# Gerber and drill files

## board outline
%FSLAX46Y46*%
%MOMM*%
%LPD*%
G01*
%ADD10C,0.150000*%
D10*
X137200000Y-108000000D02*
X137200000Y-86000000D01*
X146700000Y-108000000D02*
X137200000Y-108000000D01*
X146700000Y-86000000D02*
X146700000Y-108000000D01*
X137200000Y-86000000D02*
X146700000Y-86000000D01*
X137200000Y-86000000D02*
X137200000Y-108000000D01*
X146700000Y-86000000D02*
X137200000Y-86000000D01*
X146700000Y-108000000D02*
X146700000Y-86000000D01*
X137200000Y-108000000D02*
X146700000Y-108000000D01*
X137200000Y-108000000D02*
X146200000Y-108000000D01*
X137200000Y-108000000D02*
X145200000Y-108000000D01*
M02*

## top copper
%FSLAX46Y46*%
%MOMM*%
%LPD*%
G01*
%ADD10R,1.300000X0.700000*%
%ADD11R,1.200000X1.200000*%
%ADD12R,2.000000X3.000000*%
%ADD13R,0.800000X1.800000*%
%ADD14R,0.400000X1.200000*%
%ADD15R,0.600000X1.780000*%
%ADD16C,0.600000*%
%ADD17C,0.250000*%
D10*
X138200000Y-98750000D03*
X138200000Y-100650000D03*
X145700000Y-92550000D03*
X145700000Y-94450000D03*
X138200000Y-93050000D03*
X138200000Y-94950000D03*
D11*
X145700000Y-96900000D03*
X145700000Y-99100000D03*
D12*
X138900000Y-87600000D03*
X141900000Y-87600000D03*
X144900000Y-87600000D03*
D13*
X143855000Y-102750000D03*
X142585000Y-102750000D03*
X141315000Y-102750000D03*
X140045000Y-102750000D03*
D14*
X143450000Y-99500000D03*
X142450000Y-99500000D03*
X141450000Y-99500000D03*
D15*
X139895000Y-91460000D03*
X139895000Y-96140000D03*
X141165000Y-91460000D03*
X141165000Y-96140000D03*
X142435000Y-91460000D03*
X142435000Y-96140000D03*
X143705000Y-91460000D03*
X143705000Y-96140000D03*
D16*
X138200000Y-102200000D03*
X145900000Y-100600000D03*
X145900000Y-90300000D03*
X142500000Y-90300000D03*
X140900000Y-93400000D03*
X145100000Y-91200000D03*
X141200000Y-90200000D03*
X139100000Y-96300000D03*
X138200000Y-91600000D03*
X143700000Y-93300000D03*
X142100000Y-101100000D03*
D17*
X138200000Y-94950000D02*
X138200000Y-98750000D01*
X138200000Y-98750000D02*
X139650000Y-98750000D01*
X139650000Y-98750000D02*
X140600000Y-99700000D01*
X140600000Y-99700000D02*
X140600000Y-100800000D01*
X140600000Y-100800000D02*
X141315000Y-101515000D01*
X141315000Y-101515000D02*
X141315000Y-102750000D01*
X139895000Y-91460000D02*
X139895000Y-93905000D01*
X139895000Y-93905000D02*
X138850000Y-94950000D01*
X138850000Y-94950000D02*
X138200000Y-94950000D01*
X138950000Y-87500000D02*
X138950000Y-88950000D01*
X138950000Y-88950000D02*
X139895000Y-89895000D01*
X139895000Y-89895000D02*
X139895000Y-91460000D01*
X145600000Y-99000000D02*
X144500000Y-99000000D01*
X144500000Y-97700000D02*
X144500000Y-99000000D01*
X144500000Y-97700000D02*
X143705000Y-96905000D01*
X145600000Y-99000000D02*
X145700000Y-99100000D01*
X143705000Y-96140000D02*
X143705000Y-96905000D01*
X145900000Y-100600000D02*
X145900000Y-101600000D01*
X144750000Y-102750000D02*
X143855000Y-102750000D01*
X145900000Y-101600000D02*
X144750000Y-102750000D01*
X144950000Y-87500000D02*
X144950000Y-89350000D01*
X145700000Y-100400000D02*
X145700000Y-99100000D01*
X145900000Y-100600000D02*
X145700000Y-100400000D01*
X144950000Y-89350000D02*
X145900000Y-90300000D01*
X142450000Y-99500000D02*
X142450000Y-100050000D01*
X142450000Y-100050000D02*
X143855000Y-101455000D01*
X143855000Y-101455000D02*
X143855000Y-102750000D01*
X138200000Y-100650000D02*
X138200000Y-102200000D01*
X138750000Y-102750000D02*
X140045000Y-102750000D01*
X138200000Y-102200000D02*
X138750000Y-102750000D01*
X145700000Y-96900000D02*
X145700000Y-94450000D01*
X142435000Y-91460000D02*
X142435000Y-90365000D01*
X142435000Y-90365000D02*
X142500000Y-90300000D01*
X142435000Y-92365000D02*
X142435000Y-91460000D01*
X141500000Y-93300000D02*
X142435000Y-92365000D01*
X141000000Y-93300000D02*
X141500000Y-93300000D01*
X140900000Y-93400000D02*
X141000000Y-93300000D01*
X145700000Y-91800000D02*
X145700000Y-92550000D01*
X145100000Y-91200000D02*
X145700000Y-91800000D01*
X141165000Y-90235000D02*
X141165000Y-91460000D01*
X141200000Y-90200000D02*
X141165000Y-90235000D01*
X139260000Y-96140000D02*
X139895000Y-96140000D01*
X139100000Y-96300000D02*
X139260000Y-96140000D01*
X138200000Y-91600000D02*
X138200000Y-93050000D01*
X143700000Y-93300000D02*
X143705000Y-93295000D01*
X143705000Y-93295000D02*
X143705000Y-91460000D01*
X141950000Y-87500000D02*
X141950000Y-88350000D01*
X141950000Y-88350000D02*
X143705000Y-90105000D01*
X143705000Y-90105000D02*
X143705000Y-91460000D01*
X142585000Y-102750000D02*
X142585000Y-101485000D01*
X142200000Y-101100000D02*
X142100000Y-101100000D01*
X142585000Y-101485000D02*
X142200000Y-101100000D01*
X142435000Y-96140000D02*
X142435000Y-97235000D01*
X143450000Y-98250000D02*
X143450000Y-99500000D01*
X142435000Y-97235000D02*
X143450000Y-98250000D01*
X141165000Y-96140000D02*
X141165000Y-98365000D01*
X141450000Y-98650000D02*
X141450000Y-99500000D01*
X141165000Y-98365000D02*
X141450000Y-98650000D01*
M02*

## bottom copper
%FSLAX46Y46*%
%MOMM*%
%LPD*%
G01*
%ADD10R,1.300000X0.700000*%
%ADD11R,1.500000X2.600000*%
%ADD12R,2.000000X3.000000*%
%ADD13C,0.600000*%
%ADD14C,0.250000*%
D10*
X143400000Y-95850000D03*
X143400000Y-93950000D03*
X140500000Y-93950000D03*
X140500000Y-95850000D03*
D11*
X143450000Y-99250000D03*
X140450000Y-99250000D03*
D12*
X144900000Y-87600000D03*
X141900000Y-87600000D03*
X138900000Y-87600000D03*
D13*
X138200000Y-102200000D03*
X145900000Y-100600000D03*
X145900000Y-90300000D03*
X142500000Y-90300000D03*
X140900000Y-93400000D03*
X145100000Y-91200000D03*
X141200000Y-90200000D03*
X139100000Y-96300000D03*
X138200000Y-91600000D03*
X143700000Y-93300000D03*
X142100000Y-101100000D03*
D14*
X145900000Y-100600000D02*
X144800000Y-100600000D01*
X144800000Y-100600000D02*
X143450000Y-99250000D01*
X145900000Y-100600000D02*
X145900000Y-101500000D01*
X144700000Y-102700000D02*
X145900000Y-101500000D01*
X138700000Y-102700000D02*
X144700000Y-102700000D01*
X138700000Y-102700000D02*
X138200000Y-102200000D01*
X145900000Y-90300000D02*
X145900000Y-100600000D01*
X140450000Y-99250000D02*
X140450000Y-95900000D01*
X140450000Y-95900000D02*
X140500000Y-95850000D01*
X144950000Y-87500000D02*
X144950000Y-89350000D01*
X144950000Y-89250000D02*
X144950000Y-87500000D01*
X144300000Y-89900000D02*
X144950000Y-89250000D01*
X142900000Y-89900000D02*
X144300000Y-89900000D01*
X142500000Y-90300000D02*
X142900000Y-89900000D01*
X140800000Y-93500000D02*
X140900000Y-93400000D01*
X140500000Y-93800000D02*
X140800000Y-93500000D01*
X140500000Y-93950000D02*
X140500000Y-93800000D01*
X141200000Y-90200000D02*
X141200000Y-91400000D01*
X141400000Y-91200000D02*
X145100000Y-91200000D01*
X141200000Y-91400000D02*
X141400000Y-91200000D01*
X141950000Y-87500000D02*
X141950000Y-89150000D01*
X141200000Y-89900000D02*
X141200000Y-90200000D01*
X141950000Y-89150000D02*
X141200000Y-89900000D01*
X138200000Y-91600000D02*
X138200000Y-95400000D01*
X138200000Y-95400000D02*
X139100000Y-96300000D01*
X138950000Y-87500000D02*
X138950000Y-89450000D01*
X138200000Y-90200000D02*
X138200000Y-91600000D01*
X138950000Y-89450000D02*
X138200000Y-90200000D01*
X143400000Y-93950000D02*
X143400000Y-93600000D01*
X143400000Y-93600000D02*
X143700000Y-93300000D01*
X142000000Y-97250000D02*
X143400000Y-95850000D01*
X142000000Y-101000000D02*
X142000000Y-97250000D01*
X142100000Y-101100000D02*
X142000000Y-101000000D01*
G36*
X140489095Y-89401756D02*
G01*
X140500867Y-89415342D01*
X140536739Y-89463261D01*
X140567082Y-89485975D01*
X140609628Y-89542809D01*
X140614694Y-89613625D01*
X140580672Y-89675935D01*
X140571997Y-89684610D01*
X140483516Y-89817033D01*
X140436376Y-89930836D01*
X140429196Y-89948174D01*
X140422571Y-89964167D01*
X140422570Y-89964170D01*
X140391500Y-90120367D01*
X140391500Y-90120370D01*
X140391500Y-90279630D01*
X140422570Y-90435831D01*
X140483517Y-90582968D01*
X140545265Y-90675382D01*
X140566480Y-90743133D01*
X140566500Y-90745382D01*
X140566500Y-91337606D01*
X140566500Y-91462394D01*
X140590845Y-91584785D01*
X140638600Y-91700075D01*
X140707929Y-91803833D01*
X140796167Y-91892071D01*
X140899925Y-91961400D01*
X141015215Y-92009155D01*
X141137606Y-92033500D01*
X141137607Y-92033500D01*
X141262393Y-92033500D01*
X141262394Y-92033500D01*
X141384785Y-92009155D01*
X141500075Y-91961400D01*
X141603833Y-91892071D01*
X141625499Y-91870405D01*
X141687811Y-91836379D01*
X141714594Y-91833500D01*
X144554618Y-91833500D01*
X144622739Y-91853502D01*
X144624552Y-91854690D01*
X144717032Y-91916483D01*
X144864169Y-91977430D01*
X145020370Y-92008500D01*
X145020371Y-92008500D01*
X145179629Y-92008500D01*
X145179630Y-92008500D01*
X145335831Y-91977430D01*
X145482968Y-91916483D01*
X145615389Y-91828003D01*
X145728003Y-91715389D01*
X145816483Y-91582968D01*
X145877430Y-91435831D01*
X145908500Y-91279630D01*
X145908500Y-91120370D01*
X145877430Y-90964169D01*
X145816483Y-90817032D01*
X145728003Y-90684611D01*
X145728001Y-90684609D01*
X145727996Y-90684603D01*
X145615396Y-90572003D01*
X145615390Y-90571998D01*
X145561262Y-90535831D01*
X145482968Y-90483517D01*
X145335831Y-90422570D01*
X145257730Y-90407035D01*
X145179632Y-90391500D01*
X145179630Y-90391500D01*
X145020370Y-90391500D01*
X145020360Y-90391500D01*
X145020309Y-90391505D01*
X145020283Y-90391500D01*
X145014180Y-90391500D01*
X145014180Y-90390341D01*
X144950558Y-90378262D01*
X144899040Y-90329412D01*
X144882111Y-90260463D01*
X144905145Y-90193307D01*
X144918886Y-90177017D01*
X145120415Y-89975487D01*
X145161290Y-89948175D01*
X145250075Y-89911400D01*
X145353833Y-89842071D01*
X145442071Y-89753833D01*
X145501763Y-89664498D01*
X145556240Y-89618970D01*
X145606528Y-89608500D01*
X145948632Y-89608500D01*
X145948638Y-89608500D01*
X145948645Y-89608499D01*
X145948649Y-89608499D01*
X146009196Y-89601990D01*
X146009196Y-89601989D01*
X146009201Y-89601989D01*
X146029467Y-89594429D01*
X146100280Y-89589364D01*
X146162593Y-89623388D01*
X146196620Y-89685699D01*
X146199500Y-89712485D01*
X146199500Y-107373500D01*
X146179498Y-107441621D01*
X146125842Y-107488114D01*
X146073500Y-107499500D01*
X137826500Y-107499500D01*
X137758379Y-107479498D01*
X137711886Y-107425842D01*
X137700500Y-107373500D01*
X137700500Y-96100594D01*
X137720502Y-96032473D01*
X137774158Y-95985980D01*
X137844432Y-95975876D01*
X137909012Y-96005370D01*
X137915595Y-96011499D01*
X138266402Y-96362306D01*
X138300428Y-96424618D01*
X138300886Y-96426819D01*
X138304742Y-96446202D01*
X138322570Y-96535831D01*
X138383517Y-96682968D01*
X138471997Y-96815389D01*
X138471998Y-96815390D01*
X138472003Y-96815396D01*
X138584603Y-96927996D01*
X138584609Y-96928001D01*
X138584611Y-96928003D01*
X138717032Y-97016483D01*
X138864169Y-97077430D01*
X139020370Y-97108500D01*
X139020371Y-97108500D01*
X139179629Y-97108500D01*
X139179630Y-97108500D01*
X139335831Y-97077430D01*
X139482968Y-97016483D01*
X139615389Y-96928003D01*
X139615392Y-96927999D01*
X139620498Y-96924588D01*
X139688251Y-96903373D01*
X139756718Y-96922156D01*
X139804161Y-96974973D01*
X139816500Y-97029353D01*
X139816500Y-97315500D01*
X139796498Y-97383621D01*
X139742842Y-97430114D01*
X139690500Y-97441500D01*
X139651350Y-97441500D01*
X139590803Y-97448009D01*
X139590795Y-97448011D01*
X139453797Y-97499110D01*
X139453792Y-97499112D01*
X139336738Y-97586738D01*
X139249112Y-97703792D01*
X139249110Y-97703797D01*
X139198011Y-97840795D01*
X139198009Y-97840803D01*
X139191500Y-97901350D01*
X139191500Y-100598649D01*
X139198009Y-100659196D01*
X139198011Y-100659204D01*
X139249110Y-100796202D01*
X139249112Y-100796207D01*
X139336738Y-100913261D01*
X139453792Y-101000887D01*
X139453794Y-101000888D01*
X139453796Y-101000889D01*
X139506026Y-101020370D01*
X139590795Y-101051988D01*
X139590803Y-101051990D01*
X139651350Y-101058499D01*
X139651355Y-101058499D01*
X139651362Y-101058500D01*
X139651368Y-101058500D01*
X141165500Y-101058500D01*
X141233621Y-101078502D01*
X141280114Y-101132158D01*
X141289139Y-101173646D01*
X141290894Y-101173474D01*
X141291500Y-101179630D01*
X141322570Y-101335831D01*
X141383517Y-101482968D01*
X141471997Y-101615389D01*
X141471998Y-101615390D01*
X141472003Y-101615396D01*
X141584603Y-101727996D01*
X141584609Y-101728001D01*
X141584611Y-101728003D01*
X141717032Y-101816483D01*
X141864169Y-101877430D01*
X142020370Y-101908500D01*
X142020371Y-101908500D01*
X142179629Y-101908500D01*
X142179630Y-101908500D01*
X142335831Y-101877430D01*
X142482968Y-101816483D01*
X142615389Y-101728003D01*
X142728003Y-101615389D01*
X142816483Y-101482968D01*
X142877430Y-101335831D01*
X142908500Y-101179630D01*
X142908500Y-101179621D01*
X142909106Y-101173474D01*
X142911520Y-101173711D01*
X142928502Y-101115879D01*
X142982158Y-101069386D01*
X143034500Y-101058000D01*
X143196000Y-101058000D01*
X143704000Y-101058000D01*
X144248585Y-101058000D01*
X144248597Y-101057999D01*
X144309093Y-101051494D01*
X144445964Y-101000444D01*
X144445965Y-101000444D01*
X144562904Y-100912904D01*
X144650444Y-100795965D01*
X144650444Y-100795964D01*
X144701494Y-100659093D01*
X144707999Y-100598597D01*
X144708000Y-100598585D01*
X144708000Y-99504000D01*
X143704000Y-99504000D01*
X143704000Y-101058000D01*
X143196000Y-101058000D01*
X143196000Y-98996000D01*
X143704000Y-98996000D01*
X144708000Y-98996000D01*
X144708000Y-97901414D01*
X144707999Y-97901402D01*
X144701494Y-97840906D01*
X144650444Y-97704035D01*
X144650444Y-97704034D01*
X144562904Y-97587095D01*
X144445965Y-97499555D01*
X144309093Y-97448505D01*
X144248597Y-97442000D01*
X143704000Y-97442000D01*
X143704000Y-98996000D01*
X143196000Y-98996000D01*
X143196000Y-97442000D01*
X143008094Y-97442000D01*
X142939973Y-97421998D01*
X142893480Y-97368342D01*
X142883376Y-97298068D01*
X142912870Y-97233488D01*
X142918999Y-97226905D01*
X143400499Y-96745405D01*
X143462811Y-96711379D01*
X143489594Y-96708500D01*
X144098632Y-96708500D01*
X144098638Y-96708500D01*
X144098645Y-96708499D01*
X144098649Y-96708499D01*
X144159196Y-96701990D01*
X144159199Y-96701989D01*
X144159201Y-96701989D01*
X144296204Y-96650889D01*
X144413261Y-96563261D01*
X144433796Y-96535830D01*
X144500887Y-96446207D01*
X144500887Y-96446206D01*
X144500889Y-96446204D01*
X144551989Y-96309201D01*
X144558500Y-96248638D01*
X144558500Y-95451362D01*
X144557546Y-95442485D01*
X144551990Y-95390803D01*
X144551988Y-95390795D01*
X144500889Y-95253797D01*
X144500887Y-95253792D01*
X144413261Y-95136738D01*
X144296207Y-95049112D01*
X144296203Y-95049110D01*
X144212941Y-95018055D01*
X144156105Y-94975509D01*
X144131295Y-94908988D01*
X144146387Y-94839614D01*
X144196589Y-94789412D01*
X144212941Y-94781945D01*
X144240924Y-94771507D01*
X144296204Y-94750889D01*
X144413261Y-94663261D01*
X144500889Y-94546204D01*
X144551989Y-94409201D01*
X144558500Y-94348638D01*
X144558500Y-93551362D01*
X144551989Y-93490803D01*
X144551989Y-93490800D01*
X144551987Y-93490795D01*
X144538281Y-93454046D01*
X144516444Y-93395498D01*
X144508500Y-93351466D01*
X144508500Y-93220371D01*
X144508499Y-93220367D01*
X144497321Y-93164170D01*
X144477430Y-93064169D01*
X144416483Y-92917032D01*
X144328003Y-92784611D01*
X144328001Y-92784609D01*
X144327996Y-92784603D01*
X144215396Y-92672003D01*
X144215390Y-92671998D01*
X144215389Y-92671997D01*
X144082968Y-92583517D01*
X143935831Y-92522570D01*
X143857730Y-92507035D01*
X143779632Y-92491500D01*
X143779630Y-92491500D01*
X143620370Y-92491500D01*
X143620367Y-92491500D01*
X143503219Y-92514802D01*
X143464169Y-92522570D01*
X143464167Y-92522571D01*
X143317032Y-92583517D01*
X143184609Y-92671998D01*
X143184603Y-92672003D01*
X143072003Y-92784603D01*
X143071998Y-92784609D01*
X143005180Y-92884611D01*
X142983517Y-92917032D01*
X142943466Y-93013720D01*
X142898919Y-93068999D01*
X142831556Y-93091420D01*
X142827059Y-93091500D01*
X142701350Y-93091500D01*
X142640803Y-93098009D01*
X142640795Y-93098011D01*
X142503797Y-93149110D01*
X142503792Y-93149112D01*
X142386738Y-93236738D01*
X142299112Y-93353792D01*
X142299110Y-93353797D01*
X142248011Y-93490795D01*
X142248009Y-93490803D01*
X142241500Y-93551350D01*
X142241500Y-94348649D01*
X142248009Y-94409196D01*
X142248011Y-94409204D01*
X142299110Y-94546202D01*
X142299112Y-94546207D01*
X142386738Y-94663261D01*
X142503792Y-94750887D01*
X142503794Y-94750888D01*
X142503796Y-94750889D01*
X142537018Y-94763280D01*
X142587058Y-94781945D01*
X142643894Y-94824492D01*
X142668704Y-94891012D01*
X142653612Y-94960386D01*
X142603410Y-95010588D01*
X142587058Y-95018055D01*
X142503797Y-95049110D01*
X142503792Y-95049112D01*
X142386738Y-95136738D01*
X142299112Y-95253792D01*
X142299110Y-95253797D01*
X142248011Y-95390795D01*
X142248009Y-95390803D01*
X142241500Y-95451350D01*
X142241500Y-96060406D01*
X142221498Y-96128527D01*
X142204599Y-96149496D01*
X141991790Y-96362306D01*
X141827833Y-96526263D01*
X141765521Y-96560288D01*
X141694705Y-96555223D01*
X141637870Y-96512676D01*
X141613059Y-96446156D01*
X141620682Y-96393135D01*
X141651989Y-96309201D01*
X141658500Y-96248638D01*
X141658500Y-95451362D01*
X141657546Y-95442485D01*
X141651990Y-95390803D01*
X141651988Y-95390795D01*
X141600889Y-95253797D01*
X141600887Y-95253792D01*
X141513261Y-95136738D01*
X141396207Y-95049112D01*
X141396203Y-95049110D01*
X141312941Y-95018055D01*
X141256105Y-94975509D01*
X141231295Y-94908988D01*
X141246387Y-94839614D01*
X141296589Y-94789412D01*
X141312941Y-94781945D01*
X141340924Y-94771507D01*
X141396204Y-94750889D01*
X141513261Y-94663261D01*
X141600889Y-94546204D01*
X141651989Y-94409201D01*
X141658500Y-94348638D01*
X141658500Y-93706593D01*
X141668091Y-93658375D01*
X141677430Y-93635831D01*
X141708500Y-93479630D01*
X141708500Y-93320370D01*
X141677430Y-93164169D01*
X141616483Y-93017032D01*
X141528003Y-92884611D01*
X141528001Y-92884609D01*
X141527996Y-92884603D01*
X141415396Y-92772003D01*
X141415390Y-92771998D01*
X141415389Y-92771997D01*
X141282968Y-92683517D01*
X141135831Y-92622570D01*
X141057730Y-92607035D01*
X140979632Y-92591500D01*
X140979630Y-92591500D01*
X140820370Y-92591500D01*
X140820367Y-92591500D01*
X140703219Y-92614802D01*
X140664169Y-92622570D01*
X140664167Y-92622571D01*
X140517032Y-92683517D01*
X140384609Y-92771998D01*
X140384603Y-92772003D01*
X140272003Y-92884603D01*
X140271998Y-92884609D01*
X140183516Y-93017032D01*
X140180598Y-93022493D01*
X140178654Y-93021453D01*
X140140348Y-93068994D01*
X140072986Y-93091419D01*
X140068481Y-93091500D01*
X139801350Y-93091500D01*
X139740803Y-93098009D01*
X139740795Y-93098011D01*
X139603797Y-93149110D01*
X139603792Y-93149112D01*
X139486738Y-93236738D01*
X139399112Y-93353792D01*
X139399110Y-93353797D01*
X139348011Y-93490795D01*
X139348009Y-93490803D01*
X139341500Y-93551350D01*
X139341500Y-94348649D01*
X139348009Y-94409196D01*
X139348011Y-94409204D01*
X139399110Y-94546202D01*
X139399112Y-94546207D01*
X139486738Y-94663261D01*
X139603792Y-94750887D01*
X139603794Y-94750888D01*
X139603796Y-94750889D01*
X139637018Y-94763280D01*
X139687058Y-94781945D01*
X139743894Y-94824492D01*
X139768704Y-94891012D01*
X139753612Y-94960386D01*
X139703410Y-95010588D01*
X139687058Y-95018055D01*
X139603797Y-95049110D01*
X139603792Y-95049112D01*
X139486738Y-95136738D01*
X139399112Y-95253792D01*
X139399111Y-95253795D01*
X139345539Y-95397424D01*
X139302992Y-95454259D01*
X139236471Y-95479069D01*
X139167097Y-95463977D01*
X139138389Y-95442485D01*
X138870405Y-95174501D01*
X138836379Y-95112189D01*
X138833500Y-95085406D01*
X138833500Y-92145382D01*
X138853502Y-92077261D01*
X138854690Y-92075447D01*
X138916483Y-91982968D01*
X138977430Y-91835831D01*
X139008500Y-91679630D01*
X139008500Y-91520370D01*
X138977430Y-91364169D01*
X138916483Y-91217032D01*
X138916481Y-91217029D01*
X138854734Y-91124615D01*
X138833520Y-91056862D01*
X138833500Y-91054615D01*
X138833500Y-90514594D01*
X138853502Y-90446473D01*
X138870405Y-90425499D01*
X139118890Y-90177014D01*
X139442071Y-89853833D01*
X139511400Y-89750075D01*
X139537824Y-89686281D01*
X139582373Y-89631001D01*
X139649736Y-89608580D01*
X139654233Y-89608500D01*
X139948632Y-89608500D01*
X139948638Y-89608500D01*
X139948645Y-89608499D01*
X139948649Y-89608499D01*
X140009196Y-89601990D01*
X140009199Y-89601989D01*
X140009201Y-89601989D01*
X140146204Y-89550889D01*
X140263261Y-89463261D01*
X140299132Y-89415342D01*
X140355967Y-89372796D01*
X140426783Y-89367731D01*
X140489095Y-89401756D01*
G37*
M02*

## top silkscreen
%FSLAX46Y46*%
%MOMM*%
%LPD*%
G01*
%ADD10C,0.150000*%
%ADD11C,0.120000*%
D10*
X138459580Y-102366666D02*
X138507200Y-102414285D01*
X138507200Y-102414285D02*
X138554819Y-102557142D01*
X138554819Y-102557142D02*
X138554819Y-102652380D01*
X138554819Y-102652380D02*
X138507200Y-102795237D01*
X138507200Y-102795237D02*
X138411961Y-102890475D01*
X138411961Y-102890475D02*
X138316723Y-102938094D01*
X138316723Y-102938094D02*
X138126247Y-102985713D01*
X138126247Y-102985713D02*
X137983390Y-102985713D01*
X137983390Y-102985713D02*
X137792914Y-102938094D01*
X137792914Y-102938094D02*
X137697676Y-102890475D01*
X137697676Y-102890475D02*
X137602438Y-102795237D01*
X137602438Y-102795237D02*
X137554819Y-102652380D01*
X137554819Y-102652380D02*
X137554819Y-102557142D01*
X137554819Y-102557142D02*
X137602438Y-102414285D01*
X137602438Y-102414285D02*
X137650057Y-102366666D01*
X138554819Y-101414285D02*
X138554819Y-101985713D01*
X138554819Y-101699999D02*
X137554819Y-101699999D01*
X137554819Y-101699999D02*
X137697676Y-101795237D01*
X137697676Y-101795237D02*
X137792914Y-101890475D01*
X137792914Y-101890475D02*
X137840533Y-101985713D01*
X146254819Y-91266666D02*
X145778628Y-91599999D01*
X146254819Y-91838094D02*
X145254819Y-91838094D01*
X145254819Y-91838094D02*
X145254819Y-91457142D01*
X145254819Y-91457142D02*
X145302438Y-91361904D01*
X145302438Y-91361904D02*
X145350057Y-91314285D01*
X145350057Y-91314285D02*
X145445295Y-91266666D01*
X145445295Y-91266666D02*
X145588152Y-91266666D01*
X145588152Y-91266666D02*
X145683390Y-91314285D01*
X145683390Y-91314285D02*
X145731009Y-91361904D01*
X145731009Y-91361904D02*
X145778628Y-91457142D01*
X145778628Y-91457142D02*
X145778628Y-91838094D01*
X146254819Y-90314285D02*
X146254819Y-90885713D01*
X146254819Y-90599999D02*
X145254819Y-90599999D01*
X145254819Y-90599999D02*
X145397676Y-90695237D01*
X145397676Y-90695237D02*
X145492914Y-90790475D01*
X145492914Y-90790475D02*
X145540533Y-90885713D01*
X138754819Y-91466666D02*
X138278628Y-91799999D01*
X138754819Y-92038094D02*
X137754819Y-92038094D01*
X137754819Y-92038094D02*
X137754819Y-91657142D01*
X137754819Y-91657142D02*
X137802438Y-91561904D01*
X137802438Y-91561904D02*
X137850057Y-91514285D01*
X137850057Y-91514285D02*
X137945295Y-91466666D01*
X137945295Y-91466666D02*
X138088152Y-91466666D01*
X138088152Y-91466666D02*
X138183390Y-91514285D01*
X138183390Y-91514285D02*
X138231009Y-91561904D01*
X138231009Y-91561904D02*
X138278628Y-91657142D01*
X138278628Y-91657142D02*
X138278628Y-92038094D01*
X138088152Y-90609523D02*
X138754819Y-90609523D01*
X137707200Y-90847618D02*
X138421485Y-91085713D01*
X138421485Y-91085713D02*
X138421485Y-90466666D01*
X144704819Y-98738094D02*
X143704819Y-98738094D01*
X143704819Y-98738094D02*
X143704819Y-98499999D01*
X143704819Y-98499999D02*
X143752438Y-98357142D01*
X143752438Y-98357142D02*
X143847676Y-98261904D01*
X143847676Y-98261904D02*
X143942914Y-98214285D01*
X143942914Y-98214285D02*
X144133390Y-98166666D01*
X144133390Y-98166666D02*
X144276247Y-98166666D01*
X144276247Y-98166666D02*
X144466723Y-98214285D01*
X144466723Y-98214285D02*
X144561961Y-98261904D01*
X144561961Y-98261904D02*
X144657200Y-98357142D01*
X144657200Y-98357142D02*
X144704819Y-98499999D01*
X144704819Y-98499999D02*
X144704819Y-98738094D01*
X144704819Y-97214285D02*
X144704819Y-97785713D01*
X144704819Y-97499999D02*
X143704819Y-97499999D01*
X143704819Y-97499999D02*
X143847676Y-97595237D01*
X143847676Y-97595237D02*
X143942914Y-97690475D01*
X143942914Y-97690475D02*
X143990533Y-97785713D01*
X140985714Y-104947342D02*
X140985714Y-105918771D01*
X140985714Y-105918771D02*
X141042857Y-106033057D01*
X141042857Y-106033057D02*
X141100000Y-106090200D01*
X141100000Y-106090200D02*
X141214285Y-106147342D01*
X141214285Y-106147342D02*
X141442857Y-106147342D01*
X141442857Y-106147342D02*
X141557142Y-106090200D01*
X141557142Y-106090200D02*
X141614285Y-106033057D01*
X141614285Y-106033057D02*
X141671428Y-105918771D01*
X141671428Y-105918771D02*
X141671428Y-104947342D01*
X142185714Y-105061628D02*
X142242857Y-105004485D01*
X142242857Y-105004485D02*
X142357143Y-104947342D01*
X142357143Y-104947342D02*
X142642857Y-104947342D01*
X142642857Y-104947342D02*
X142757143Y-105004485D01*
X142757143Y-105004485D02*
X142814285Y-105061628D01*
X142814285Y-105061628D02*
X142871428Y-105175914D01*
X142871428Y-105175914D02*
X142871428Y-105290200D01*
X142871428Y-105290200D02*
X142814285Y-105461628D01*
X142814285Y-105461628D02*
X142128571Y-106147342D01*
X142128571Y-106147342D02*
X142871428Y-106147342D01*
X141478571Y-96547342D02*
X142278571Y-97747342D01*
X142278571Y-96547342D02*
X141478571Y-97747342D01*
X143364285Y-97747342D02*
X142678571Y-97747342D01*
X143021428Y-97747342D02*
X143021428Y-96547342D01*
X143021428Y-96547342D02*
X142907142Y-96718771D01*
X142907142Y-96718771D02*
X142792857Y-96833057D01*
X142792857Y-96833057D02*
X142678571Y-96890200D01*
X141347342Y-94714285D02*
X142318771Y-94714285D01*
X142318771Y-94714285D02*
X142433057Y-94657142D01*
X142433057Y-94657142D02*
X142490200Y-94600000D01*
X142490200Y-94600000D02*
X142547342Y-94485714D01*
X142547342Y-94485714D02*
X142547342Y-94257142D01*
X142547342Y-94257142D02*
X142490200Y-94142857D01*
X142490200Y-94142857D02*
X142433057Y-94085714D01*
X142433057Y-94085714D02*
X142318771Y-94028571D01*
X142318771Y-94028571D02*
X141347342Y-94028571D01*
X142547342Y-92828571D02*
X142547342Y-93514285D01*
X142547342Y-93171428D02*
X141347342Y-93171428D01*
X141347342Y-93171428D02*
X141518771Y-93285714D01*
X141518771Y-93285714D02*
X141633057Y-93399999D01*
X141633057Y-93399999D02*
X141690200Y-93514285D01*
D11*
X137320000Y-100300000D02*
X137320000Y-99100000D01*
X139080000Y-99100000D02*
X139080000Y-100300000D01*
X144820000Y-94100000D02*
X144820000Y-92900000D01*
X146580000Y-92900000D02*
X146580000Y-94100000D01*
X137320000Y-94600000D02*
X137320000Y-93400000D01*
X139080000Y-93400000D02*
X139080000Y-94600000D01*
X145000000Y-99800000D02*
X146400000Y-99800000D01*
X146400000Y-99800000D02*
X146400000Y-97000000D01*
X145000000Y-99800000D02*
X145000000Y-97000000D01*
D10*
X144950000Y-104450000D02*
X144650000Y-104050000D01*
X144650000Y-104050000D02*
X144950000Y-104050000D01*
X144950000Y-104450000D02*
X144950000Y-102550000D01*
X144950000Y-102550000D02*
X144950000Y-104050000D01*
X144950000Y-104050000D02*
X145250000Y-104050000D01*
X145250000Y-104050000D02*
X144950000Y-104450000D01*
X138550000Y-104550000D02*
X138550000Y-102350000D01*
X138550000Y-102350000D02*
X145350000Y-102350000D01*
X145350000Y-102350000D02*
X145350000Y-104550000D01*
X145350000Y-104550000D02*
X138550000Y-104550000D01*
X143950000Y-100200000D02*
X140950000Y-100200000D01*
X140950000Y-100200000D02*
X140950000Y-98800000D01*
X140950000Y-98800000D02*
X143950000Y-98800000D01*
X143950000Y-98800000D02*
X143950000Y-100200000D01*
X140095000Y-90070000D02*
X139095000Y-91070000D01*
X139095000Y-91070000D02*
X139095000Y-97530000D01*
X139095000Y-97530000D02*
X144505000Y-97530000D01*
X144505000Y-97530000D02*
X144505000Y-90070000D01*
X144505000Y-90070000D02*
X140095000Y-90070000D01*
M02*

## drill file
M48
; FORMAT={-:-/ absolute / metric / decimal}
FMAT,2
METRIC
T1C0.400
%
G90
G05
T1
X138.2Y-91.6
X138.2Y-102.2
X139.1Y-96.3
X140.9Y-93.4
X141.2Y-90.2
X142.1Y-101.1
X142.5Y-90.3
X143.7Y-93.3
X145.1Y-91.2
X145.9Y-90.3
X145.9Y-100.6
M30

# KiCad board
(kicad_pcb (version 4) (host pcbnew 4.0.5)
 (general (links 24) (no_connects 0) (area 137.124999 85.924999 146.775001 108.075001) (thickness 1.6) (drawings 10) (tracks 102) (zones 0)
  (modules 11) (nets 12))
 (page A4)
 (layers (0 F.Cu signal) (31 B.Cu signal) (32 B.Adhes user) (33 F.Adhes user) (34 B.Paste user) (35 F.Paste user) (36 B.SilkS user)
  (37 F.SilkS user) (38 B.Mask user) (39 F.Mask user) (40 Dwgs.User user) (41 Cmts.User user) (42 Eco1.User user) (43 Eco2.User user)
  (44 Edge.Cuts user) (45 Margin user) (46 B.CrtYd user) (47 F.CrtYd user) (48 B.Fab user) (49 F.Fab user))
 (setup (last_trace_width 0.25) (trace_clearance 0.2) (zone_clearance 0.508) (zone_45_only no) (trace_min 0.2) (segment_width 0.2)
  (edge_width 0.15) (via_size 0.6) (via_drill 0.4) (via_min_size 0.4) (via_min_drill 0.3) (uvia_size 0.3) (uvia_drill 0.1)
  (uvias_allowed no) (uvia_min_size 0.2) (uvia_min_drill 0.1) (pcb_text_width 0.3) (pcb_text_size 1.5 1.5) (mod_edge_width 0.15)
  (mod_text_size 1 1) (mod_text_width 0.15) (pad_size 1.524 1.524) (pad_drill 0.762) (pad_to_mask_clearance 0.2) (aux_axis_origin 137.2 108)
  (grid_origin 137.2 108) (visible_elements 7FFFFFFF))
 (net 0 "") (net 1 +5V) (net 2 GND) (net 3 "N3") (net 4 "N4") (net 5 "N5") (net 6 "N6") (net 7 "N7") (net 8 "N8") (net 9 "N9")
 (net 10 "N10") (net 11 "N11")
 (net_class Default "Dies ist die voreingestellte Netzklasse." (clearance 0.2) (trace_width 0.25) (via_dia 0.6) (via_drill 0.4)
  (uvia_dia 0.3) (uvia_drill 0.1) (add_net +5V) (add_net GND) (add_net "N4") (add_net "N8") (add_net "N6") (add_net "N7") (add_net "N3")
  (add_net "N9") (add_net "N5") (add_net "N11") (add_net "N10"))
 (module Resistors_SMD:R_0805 (layer F.Cu) (at 138.2 99.7 270)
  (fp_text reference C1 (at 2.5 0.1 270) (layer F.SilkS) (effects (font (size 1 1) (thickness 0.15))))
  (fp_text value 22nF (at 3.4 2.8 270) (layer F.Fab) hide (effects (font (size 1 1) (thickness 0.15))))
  (fp_line (start 0.6 0.88) (end -0.6 0.88) (layer F.SilkS) (width 0.12))
  (fp_line (start -0.6 -0.88) (end 0.6 -0.88) (layer F.SilkS) (width 0.12))
  (pad 1 smd rect (at -0.95 0 270) (size 0.7 1.3) (layers F.Cu F.Paste F.Mask) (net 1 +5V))
  (pad 2 smd rect (at 0.95 0 270) (size 0.7 1.3) (layers F.Cu F.Paste F.Mask) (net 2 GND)))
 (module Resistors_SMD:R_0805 (layer F.Cu) (at 145.7 93.5 270)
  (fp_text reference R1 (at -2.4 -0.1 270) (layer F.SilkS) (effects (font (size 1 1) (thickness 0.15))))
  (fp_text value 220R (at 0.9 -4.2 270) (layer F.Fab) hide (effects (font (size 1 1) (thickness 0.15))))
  (fp_line (start 0.6 0.88) (end -0.6 0.88) (layer F.SilkS) (width 0.12))
  (fp_line (start -0.6 -0.88) (end 0.6 -0.88) (layer F.SilkS) (width 0.12))
  (pad 1 smd rect (at -0.95 0 270) (size 0.7 1.3) (layers F.Cu F.Paste F.Mask) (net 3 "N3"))
  (pad 2 smd rect (at 0.95 0 270) (size 0.7 1.3) (layers F.Cu F.Paste F.Mask) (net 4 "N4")))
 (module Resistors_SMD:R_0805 (layer B.Cu) (at 143.4 94.9 90)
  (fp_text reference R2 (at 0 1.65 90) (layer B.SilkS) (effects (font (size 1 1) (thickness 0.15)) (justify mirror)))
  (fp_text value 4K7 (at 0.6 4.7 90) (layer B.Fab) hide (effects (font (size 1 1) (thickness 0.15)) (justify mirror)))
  (pad 1 smd rect (at -0.95 0 90) (size 0.7 1.3) (layers B.Cu B.Paste B.Mask) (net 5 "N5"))
  (pad 2 smd rect (at 0.95 0 90) (size 0.7 1.3) (layers B.Cu B.Paste B.Mask) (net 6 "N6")))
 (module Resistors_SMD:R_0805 (layer B.Cu) (at 140.5 94.9 270)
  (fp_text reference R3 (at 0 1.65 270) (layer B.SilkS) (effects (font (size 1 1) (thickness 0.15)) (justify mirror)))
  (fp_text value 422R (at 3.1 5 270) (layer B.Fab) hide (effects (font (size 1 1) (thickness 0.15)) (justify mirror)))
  (pad 1 smd rect (at -0.95 0 270) (size 0.7 1.3) (layers B.Cu B.Paste B.Mask) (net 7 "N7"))
  (pad 2 smd rect (at 0.95 0 270) (size 0.7 1.3) (layers B.Cu B.Paste B.Mask) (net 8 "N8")))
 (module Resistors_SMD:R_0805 (layer F.Cu) (at 138.2 94 270)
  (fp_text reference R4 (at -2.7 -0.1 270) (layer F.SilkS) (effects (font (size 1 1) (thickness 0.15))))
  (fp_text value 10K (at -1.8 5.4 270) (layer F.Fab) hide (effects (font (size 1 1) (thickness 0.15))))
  (fp_line (start 0.6 0.88) (end -0.6 0.88) (layer F.SilkS) (width 0.12))
  (fp_line (start -0.6 -0.88) (end 0.6 -0.88) (layer F.SilkS) (width 0.12))
  (pad 1 smd rect (at -0.95 0 270) (size 0.7 1.3) (layers F.Cu F.Paste F.Mask) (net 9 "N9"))
  (pad 2 smd rect (at 0.95 0 270) (size 0.7 1.3) (layers F.Cu F.Paste F.Mask) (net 1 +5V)))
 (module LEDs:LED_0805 (layer F.Cu) (at 145.7 98 90)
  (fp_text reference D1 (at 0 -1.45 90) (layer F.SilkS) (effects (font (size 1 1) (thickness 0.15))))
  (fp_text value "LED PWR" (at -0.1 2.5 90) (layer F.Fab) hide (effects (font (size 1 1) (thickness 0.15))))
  (fp_line (start -1.8 -0.7) (end -1.8 0.7) (layer F.SilkS) (width 0.12))
  (fp_line (start -1.8 0.7) (end 1 0.7) (layer F.SilkS) (width 0.12))
  (fp_line (start -1.8 -0.7) (end 1 -0.7) (layer F.SilkS) (width 0.12))
  (pad 2 smd rect (at 1.1 0 270) (size 1.2 1.2) (layers F.Cu F.Paste F.Mask) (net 4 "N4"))
  (pad 1 smd rect (at -1.1 0 270) (size 1.2 1.2) (layers F.Cu F.Paste F.Mask) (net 2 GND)))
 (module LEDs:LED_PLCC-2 (layer B.Cu) (at 141.95 99.25 180)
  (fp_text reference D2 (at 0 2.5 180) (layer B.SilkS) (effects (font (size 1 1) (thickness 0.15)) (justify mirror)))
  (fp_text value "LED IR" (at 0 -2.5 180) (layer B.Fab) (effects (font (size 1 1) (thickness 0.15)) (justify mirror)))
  (pad 1 smd rect (at -1.5 0 180) (size 1.5 2.6) (layers B.Cu B.Paste B.Mask) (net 2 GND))
  (pad 2 smd rect (at 1.5 0 180) (size 1.5 2.6) (layers B.Cu B.Paste B.Mask) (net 8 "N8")))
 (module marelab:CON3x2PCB (layer F.Cu) (at 141.9 87.6)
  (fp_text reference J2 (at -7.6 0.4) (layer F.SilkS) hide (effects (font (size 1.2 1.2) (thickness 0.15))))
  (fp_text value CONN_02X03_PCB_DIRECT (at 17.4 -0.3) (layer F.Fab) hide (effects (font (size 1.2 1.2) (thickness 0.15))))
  (pad 4 smd rect (at 3 0) (size 2 3) (layers *.Mask B.Cu B.Paste) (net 7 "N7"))
  (pad 5 smd rect (at 0 0) (size 2 3) (layers B.Cu F.Paste B.Mask) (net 3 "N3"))
  (pad 6 smd rect (at -3 0) (size 2 3) (layers B.Cu B.Paste B.Mask) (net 9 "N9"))
  (pad 1 smd rect (at -3 0) (size 2 3) (layers F.Cu F.Paste F.Mask) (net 1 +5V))
  (pad 2 smd rect (at 0 0) (size 2 3) (layers F.Cu F.Paste F.Mask) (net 6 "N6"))
  (pad 3 smd rect (at 3 0) (size 2 3) (layers F.Cu F.Paste F.Mask) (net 2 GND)))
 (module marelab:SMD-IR (layer F.Cu) (at 141.95 102.75 180)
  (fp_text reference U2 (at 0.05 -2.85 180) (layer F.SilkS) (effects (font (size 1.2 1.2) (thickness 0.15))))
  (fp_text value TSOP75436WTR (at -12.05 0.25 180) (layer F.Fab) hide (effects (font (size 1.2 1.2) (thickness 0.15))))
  (fp_line (start -3 -1.7) (end -2.7 -1.3) (layer F.SilkS) (width 0.15))
  (fp_line (start -2.7 -1.3) (end -3 -1.3) (layer F.SilkS) (width 0.15))
  (fp_line (start -3 -1.7) (end -3 0.2) (layer F.SilkS) (width 0.15))
  (fp_line (start -3 0.2) (end -3 -1.3) (layer F.SilkS) (width 0.15))
  (fp_line (start -3 -1.3) (end -3.3 -1.3) (layer F.SilkS) (width 0.15))
  (fp_line (start -3.3 -1.3) (end -3 -1.7) (layer F.SilkS) (width 0.15))
  (fp_line (start 3.4 -1.8) (end 3.4 0.4) (layer F.SilkS) (width 0.15))
  (fp_line (start 3.4 0.4) (end -3.4 0.4) (layer F.SilkS) (width 0.15))
  (fp_line (start -3.4 0.4) (end -3.4 -1.8) (layer F.SilkS) (width 0.15))
  (fp_line (start -3.4 -1.8) (end 3.4 -1.8) (layer F.SilkS) (width 0.15))
  (pad 4 smd rect (at -1.905 0 180) (size 0.8 1.8) (layers F.Cu F.Paste F.Mask) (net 2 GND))
  (pad 3 smd rect (at -0.635 0 180) (size 0.8 1.8) (layers F.Cu F.Paste F.Mask) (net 5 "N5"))
  (pad 2 smd rect (at 0.635 0 180) (size 0.8 1.8) (layers F.Cu F.Paste F.Mask) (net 1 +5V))
  (pad 1 smd rect (at 1.905 0 180) (size 0.8 1.8) (layers F.Cu F.Paste F.Mask) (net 2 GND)))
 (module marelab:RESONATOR (layer F.Cu) (at 142.45 99.5 180)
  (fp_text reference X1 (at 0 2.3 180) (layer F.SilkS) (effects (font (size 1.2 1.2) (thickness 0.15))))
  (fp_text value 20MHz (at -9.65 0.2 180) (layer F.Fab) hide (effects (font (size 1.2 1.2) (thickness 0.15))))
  (fp_line (start -1.5 -0.7) (end 1.5 -0.7) (layer F.SilkS) (width 0.15))
  (fp_line (start 1.5 -0.7) (end 1.5 0.7) (layer F.SilkS) (width 0.15))
  (fp_line (start 1.5 0.7) (end -1.5 0.7) (layer F.SilkS) (width 0.15))
  (fp_line (start -1.5 0.7) (end -1.5 -0.7) (layer F.SilkS) (width 0.15))
  (pad 1 smd rect (at -1 0 180) (size 0.4 1.2) (layers F.Cu F.Paste F.Mask) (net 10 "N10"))
  (pad 2 smd rect (at 0 0 180) (size 0.4 1.2) (layers F.Cu F.Paste F.Mask) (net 2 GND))
  (pad 3 smd rect (at 1 0 180) (size 0.4 1.2) (layers F.Cu F.Paste F.Mask) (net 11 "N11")))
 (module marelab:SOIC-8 (layer F.Cu) (at 141.8 93.8)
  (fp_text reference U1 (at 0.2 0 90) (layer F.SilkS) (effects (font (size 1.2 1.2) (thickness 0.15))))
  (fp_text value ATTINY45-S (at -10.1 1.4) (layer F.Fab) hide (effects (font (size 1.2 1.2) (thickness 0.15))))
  (fp_line (start -1.705 -3.73) (end -2.705 -2.73) (layer F.SilkS) (width 0.15))
  (fp_line (start -2.705 -2.73) (end -2.705 3.73) (layer F.SilkS) (width 0.15))
  (fp_line (start -2.705 3.73) (end 2.705 3.73) (layer F.SilkS) (width 0.15))
  (fp_line (start 2.705 3.73) (end 2.705 -3.73) (layer F.SilkS) (width 0.15))
  (fp_line (start 2.705 -3.73) (end -1.705 -3.73) (layer F.SilkS) (width 0.15))
  (pad 8 smd rect (at -1.905 -2.34) (size 0.6 1.78) (layers F.Cu F.Paste F.Mask) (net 1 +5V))
  (pad 1 smd rect (at -1.905 2.34) (size 0.6 1.78) (layers F.Cu F.Paste F.Mask) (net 9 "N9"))
  (pad 7 smd rect (at -0.635 -2.34) (size 0.6 1.78) (layers F.Cu F.Paste F.Mask) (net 3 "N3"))
  (pad 2 smd rect (at -0.635 2.34) (size 0.6 1.78) (layers F.Cu F.Paste F.Mask) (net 11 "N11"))
  (pad 6 smd rect (at 0.635 -2.34) (size 0.6 1.78) (layers F.Cu F.Paste F.Mask) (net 7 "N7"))
  (pad 3 smd rect (at 0.635 2.34) (size 0.6 1.78) (layers F.Cu F.Paste F.Mask) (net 10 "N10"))
  (pad 5 smd rect (at 1.905 -2.34) (size 0.6 1.78) (layers F.Cu F.Paste F.Mask) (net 6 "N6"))
  (pad 4 smd rect (at 1.905 2.34) (size 0.6 1.78) (layers F.Cu F.Paste F.Mask) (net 2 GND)))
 (gr_line (start 137.2 108) (end 137.2 86) (angle 90) (layer Edge.Cuts) (width 0.15))
 (gr_line (start 146.7 108) (end 137.2 108) (angle 90) (layer Edge.Cuts) (width 0.15))
 (gr_line (start 146.7 86) (end 146.7 108) (angle 90) (layer Edge.Cuts) (width 0.15))
 (gr_line (start 137.2 86) (end 146.7 86) (angle 90) (layer Edge.Cuts) (width 0.15))
 (gr_line (start 137.2 86) (end 137.2 108) (angle 90) (layer Edge.Cuts) (width 0.15))
 (gr_line (start 146.7 86) (end 137.2 86) (angle 90) (layer Edge.Cuts) (width 0.15))
 (gr_line (start 146.7 108) (end 146.7 86) (angle 90) (layer Edge.Cuts) (width 0.15))
 (gr_line (start 137.2 108) (end 146.7 108) (angle 90) (layer Edge.Cuts) (width 0.15))
 (gr_line (start 137.2 108) (end 146.2 108) (angle 90) (layer Edge.Cuts) (width 0.15))
 (gr_line (start 137.2 108) (end 145.2 108) (angle 90) (layer Edge.Cuts) (width 0.15))
 (segment (start 138.2 94.95) (end 138.2 98.75) (width 0.25) (layer F.Cu) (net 1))
 (segment (start 138.2 98.75) (end 139.65 98.75) (width 0.25) (layer F.Cu) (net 1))
 (segment (start 139.65 98.75) (end 140.6 99.7) (width 0.25) (layer F.Cu) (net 1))
 (segment (start 140.6 99.7) (end 140.6 100.8) (width 0.25) (layer F.Cu) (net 1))
 (segment (start 140.6 100.8) (end 141.315 101.515) (width 0.25) (layer F.Cu) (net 1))
 (segment (start 141.315 101.515) (end 141.315 102.75) (width 0.25) (layer F.Cu) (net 1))
 (segment (start 139.895 91.46) (end 139.895 93.905) (width 0.25) (layer F.Cu) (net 1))
 (segment (start 139.895 93.905) (end 138.85 94.95) (width 0.25) (layer F.Cu) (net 1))
 (segment (start 138.85 94.95) (end 138.2 94.95) (width 0.25) (layer F.Cu) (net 1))
 (segment (start 138.95 87.5) (end 138.95 88.95) (width 0.25) (layer F.Cu) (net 1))
 (segment (start 138.95 88.95) (end 139.895 89.895) (width 0.25) (layer F.Cu) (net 1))
 (segment (start 139.895 89.895) (end 139.895 91.46) (width 0.25) (layer F.Cu) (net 1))
 (segment (start 145.6 99) (end 144.5 99) (width 0.25) (layer F.Cu) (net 2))
 (segment (start 144.5 97.7) (end 144.5 99) (width 0.25) (layer F.Cu) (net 2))
 (segment (start 144.5 97.7) (end 143.705 96.905) (width 0.25) (layer F.Cu) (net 2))
 (segment (start 145.6 99) (end 145.7 99.1) (width 0.25) (layer F.Cu) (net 2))
 (segment (start 143.705 96.14) (end 143.705 96.905) (width 0.25) (layer F.Cu) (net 2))
 (segment (start 145.9 100.6) (end 144.8 100.6) (width 0.25) (layer B.Cu) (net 2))
 (segment (start 144.8 100.6) (end 143.45 99.25) (width 0.25) (layer B.Cu) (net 2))
 (via (at 138.2 102.2) (size 0.6) (drill 0.4) (layers F.Cu B.Cu) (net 2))
 (segment (start 145.9 100.6) (end 145.9 101.5) (width 0.25) (layer B.Cu) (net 2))
 (segment (start 144.7 102.7) (end 145.9 101.5) (width 0.25) (layer B.Cu) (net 2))
 (segment (start 138.7 102.7) (end 144.7 102.7) (width 0.25) (layer B.Cu) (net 2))
 (segment (start 138.7 102.7) (end 138.2 102.2) (width 0.25) (layer B.Cu) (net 2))
 (segment (start 145.9 100.6) (end 145.9 101.6) (width 0.25) (layer F.Cu) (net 2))
 (segment (start 144.75 102.75) (end 143.855 102.75) (width 0.25) (layer F.Cu) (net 2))
 (segment (start 145.9 101.6) (end 144.75 102.75) (width 0.25) (layer F.Cu) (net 2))
 (segment (start 144.95 87.5) (end 144.95 89.35) (width 0.25) (layer F.Cu) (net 2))
 (segment (start 145.7 100.4) (end 145.7 99.1) (width 0.25) (layer F.Cu) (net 2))
 (segment (start 145.9 100.6) (end 145.7 100.4) (width 0.25) (layer F.Cu) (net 2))
 (via (at 145.9 100.6) (size 0.6) (drill 0.4) (layers F.Cu B.Cu) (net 2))
 (segment (start 145.9 90.3) (end 145.9 100.6) (width 0.25) (layer B.Cu) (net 2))
 (via (at 145.9 90.3) (size 0.6) (drill 0.4) (layers F.Cu B.Cu) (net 2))
 (segment (start 144.95 89.35) (end 145.9 90.3) (width 0.25) (layer F.Cu) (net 2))
 (segment (start 142.45 99.5) (end 142.45 100.05) (width 0.25) (layer F.Cu) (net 2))
 (segment (start 142.45 100.05) (end 143.855 101.455) (width 0.25) (layer F.Cu) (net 2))
 (segment (start 143.855 101.455) (end 143.855 102.75) (width 0.25) (layer F.Cu) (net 2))
 (segment (start 138.2 100.65) (end 138.2 102.2) (width 0.25) (layer F.Cu) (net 2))
 (segment (start 138.75 102.75) (end 140.045 102.75) (width 0.25) (layer F.Cu) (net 2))
 (segment (start 138.2 102.2) (end 138.75 102.75) (width 0.25) (layer F.Cu) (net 2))
 (segment (start 145.7 96.9) (end 145.7 94.45) (width 0.25) (layer F.Cu) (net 4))
 (segment (start 140.45 99.25) (end 140.45 95.9) (width 0.25) (layer B.Cu) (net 8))
 (segment (start 140.45 95.9) (end 140.5 95.85) (width 0.25) (layer B.Cu) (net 8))
 (segment (start 144.95 87.5) (end 144.95 89.35) (width 0.25) (layer B.Cu) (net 7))
 (segment (start 142.435 91.46) (end 142.435 90.365) (width 0.25) (layer F.Cu) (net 7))
 (segment (start 144.95 89.25) (end 144.95 87.5) (width 0.25) (layer B.Cu) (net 7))
 (segment (start 144.3 89.9) (end 144.95 89.25) (width 0.25) (layer B.Cu) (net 7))
 (segment (start 142.9 89.9) (end 144.3 89.9) (width 0.25) (layer B.Cu) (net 7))
 (segment (start 142.5 90.3) (end 142.9 89.9) (width 0.25) (layer B.Cu) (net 7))
 (via (at 142.5 90.3) (size 0.6) (drill 0.4) (layers F.Cu B.Cu) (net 7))
 (segment (start 142.435 90.365) (end 142.5 90.3) (width 0.25) (layer F.Cu) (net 7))
 (segment (start 140.8 93.5) (end 140.9 93.4) (width 0.25) (layer B.Cu) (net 7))
 (segment (start 140.5 93.8) (end 140.8 93.5) (width 0.25) (layer B.Cu) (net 7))
 (segment (start 142.435 92.365) (end 142.435 91.46) (width 0.25) (layer F.Cu) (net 7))
 (segment (start 141.5 93.3) (end 142.435 92.365) (width 0.25) (layer F.Cu) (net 7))
 (segment (start 141 93.3) (end 141.5 93.3) (width 0.25) (layer F.Cu) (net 7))
 (segment (start 140.9 93.4) (end 141 93.3) (width 0.25) (layer F.Cu) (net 7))
 (via (at 140.9 93.4) (size 0.6) (drill 0.4) (layers F.Cu B.Cu) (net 7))
 (segment (start 140.5 93.95) (end 140.5 93.8) (width 0.25) (layer B.Cu) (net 7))
 (segment (start 141.2 90.2) (end 141.2 91.4) (width 0.25) (layer B.Cu) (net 3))
 (segment (start 145.7 91.8) (end 145.7 92.55) (width 0.25) (layer F.Cu) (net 3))
 (segment (start 145.1 91.2) (end 145.7 91.8) (width 0.25) (layer F.Cu) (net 3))
 (via (at 145.1 91.2) (size 0.6) (drill 0.4) (layers F.Cu B.Cu) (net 3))
 (segment (start 141.4 91.2) (end 145.1 91.2) (width 0.25) (layer B.Cu) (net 3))
 (segment (start 141.2 91.4) (end 141.4 91.2) (width 0.25) (layer B.Cu) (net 3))
 (segment (start 141.95 87.5) (end 141.95 89.15) (width 0.25) (layer B.Cu) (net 3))
 (segment (start 141.165 90.235) (end 141.165 91.46) (width 0.25) (layer F.Cu) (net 3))
 (segment (start 141.2 90.2) (end 141.165 90.235) (width 0.25) (layer F.Cu) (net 3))
 (via (at 141.2 90.2) (size 0.6) (drill 0.4) (layers F.Cu B.Cu) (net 3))
 (segment (start 141.2 89.9) (end 141.2 90.2) (width 0.25) (layer B.Cu) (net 3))
 (segment (start 141.95 89.15) (end 141.2 89.9) (width 0.25) (layer B.Cu) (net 3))
 (segment (start 138.2 91.6) (end 138.2 95.4) (width 0.25) (layer B.Cu) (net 9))
 (segment (start 139.26 96.14) (end 139.895 96.14) (width 0.25) (layer F.Cu) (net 9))
 (segment (start 139.1 96.3) (end 139.26 96.14) (width 0.25) (layer F.Cu) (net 9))
 (via (at 139.1 96.3) (size 0.6) (drill 0.4) (layers F.Cu B.Cu) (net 9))
 (segment (start 138.2 95.4) (end 139.1 96.3) (width 0.25) (layer B.Cu) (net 9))
 (segment (start 138.95 87.5) (end 138.95 89.45) (width 0.25) (layer B.Cu) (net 9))
 (segment (start 138.2 91.6) (end 138.2 93.05) (width 0.25) (layer F.Cu) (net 9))
 (via (at 138.2 91.6) (size 0.6) (drill 0.4) (layers F.Cu B.Cu) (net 9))
 (segment (start 138.2 90.2) (end 138.2 91.6) (width 0.25) (layer B.Cu) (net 9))
 (segment (start 138.95 89.45) (end 138.2 90.2) (width 0.25) (layer B.Cu) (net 9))
 (segment (start 143.4 93.95) (end 143.4 93.6) (width 0.25) (layer B.Cu) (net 6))
 (segment (start 143.4 93.6) (end 143.7 93.3) (width 0.25) (layer B.Cu) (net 6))
 (via (at 143.7 93.3) (size 0.6) (drill 0.4) (layers F.Cu B.Cu) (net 6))
 (segment (start 143.7 93.3) (end 143.705 93.295) (width 0.25) (layer F.Cu) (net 6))
 (segment (start 143.705 93.295) (end 143.705 91.46) (width 0.25) (layer F.Cu) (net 6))
 (segment (start 141.95 87.5) (end 141.95 88.35) (width 0.25) (layer F.Cu) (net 6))
 (segment (start 141.95 88.35) (end 143.705 90.105) (width 0.25) (layer F.Cu) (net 6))
 (segment (start 143.705 90.105) (end 143.705 91.46) (width 0.25) (layer F.Cu) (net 6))
 (segment (start 142.585 102.75) (end 142.585 101.485) (width 0.25) (layer F.Cu) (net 5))
 (segment (start 142 97.25) (end 143.4 95.85) (width 0.25) (layer B.Cu) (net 5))
 (segment (start 142 101) (end 142 97.25) (width 0.25) (layer B.Cu) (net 5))
 (segment (start 142.1 101.1) (end 142 101) (width 0.25) (layer B.Cu) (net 5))
 (via (at 142.1 101.1) (size 0.6) (drill 0.4) (layers F.Cu B.Cu) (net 5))
 (segment (start 142.2 101.1) (end 142.1 101.1) (width 0.25) (layer F.Cu) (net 5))
 (segment (start 142.585 101.485) (end 142.2 101.1) (width 0.25) (layer F.Cu) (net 5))
 (segment (start 142.435 96.14) (end 142.435 97.235) (width 0.25) (layer F.Cu) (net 10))
 (segment (start 143.45 98.25) (end 143.45 99.5) (width 0.25) (layer F.Cu) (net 10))
 (segment (start 142.435 97.235) (end 143.45 98.25) (width 0.25) (layer F.Cu) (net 10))
 (segment (start 141.165 96.14) (end 141.165 98.365) (width 0.25) (layer F.Cu) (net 11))
 (segment (start 141.45 98.65) (end 141.45 99.5) (width 0.25) (layer F.Cu) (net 11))
 (segment (start 141.165 98.365) (end 141.45 98.65) (width 0.25) (layer F.Cu) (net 11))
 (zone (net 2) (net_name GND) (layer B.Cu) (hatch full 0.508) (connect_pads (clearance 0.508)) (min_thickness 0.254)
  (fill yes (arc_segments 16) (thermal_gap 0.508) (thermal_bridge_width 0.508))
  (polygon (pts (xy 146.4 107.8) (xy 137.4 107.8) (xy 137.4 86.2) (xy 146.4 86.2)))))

